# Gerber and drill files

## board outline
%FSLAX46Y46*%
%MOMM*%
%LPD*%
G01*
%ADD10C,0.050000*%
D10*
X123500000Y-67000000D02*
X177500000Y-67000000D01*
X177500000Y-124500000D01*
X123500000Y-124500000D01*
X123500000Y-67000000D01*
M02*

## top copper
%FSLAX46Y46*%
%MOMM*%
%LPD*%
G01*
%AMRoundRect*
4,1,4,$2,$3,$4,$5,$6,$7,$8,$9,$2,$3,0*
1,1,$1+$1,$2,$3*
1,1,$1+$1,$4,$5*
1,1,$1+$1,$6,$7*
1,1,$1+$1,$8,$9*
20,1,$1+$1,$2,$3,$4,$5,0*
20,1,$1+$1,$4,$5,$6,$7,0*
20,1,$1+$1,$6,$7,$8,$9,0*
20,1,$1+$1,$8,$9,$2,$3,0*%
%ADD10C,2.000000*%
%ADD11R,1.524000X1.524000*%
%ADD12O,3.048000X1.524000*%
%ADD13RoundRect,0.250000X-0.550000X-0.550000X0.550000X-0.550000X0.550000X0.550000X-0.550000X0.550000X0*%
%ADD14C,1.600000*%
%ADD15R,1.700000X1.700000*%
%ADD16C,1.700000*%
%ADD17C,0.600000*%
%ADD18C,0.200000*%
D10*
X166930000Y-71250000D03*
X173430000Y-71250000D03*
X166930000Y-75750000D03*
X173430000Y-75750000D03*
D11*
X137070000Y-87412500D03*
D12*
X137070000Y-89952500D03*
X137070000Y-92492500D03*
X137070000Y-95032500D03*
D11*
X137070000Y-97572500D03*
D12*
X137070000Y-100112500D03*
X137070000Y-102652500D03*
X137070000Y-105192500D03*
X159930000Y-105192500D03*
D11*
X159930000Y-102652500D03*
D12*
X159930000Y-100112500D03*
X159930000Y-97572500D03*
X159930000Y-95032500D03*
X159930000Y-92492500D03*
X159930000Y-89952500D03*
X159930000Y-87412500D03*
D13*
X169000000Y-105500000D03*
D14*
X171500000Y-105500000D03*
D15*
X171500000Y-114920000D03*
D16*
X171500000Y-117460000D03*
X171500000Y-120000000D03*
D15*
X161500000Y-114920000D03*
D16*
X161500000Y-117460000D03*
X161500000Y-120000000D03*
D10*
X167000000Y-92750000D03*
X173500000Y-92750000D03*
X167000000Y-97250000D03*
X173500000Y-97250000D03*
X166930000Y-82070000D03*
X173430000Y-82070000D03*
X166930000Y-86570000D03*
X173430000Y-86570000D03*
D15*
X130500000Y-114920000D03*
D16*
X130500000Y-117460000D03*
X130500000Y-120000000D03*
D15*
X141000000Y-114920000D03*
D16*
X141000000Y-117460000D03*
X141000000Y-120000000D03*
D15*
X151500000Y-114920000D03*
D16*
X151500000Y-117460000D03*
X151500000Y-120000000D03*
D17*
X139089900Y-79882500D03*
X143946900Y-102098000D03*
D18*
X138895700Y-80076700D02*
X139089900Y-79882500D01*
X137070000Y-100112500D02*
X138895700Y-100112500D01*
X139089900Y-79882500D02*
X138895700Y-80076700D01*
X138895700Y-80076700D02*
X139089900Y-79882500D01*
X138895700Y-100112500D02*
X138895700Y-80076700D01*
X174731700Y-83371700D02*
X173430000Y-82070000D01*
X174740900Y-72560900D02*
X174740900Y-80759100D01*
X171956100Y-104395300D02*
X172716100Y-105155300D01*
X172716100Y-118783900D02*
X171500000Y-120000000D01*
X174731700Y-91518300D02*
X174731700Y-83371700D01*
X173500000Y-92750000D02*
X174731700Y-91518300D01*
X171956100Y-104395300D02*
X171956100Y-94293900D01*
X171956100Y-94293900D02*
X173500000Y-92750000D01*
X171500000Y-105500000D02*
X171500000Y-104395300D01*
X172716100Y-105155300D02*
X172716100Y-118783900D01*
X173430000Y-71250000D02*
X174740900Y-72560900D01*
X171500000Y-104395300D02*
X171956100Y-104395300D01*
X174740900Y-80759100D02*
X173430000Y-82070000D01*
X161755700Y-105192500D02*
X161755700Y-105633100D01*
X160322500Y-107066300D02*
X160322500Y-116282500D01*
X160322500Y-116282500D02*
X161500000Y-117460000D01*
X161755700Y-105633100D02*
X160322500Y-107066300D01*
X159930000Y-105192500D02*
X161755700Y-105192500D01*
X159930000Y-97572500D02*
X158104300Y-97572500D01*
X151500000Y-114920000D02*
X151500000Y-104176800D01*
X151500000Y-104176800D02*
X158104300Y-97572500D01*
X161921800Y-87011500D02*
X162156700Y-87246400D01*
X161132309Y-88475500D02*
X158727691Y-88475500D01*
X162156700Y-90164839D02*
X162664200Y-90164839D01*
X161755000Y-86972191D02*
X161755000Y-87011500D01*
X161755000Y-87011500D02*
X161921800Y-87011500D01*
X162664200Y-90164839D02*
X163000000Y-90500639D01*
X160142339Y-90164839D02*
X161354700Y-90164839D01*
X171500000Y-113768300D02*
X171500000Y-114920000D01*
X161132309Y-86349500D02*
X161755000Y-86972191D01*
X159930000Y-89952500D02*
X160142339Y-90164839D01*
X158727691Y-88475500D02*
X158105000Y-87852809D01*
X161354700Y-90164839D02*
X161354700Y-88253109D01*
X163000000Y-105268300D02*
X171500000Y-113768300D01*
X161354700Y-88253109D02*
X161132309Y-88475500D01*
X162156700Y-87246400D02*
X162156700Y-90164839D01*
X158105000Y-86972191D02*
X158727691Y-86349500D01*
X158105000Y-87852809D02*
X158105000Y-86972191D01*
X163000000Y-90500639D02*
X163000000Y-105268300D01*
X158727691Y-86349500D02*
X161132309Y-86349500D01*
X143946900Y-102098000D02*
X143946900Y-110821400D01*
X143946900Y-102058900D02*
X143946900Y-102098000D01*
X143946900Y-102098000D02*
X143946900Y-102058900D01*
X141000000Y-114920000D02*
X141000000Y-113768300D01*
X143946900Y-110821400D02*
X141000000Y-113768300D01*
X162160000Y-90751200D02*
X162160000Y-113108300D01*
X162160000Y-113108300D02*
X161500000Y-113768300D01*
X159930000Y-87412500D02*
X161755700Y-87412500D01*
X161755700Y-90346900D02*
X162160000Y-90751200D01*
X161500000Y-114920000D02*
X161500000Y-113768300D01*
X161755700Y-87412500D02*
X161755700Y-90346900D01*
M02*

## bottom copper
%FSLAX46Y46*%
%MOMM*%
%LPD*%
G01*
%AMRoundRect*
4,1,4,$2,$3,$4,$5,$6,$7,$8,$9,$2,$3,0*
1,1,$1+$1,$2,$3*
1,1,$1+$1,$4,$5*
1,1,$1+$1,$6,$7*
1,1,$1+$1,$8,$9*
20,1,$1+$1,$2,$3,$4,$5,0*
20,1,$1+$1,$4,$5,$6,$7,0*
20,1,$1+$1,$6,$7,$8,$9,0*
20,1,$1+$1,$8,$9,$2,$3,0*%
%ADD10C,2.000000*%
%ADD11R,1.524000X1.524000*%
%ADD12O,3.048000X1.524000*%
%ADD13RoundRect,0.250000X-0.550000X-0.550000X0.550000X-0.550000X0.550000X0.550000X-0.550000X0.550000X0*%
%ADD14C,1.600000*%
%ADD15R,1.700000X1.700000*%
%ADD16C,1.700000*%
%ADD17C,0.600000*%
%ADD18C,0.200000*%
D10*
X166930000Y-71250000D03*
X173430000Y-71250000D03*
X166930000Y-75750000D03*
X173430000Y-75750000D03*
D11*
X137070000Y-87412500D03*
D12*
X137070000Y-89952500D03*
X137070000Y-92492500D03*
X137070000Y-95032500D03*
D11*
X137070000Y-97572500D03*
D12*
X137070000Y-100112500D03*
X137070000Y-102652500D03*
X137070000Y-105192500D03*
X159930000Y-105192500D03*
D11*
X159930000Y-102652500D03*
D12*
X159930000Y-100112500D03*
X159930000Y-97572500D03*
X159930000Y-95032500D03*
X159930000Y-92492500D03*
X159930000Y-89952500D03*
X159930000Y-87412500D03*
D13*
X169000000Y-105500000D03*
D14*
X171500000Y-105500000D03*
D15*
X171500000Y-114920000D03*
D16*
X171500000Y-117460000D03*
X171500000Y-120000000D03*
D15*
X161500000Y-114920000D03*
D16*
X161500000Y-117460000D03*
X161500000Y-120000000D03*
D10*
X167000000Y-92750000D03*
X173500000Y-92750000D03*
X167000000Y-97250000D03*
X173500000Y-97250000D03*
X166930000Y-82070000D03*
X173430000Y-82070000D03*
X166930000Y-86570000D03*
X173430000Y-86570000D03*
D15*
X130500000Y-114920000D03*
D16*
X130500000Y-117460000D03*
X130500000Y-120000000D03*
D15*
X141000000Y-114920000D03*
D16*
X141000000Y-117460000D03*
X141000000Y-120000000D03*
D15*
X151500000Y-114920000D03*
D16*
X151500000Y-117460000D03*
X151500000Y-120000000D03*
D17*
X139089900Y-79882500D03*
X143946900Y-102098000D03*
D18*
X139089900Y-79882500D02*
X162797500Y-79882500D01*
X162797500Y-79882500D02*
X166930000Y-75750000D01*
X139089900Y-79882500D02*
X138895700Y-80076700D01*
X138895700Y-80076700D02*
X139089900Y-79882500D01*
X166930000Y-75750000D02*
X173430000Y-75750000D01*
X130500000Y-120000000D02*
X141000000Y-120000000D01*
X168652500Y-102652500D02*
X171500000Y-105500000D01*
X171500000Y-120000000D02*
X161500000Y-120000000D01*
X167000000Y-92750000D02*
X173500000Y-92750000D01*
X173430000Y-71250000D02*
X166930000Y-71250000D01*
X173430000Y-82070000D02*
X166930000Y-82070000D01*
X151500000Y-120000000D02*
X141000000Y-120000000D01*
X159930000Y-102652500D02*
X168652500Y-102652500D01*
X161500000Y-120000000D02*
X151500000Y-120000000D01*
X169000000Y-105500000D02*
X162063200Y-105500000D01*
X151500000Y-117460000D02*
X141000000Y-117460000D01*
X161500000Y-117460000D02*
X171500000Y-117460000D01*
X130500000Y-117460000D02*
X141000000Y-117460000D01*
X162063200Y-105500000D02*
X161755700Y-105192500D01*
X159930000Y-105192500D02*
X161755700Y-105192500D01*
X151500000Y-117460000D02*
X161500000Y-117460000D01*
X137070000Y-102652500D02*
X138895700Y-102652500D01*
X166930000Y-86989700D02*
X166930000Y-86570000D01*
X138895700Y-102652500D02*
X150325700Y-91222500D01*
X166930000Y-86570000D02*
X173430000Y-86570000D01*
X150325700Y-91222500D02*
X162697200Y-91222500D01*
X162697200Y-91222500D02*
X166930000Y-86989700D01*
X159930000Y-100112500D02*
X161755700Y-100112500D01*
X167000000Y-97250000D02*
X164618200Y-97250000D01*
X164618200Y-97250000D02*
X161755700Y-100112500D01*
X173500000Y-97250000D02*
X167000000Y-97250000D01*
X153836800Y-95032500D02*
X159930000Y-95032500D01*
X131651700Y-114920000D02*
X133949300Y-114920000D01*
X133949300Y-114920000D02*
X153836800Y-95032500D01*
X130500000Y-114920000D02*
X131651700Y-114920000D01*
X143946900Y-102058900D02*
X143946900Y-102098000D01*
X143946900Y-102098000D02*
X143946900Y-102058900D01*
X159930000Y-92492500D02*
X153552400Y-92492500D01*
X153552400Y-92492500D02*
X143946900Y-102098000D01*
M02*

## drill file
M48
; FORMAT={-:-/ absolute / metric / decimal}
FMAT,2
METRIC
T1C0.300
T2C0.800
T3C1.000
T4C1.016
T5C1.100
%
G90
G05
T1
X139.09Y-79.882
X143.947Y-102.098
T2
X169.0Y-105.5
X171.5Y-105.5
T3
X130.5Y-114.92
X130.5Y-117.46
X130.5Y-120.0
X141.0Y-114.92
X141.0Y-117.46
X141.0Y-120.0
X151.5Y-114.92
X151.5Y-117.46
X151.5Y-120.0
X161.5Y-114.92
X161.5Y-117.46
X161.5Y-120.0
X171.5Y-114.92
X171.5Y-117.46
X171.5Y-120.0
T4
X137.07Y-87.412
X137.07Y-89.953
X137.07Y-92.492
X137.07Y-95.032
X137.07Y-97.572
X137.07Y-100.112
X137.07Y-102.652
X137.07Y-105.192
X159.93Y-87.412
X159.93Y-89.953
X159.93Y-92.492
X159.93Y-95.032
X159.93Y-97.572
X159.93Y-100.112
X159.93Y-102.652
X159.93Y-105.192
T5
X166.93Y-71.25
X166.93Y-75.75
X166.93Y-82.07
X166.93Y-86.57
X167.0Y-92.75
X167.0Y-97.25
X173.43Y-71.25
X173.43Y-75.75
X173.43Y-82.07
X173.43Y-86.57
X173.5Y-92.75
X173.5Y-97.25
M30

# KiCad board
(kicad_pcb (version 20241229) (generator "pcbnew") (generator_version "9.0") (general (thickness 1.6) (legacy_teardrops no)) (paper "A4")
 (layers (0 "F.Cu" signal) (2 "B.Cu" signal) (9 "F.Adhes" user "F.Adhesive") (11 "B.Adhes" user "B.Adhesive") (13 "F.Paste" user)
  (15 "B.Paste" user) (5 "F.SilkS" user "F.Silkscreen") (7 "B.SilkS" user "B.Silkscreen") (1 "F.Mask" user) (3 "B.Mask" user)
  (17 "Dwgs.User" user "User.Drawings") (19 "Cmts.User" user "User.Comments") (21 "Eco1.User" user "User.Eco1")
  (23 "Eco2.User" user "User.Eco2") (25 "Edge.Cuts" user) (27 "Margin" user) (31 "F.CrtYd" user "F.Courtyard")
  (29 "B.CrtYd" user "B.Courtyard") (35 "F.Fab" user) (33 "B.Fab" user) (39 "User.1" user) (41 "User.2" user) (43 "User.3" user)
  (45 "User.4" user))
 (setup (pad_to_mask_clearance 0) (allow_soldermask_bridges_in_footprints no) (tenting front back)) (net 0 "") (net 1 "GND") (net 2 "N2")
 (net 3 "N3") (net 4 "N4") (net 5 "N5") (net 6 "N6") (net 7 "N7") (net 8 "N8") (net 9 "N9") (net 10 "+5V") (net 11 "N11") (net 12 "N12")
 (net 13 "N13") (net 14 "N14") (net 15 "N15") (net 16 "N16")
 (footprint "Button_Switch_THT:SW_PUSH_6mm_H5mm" (layer "F.Cu") (at 166.93 71.25)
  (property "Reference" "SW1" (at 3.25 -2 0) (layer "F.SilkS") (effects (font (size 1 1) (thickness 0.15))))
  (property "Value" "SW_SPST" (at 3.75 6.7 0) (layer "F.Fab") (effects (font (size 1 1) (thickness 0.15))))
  (pad "1" thru_hole circle (at 0 0 90) (size 2 2) (drill 1.1) (layers "*.Cu" "*.Mask") (remove_unused_layers no) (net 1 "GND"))
  (pad "1" thru_hole circle (at 6.5 0 90) (size 2 2) (drill 1.1) (layers "*.Cu" "*.Mask") (remove_unused_layers no) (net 1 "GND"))
  (pad "2" thru_hole circle (at 0 4.5 90) (size 2 2) (drill 1.1) (layers "*.Cu" "*.Mask") (remove_unused_layers no) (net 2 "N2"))
  (pad "2" thru_hole circle (at 6.5 4.5 90) (size 2 2) (drill 1.1) (layers "*.Cu" "*.Mask") (remove_unused_layers no) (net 2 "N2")))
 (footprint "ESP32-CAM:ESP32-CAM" (layer "F.Cu") (at 148.5 95.0325)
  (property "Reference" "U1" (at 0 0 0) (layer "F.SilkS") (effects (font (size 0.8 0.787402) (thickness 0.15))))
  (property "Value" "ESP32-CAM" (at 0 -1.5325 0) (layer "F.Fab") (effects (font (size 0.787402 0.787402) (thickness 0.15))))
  (pad "P$1" thru_hole rect (at -11.43 -7.62) (size 1.524 1.524) (drill 1.016) (layers "*.Cu" "*.Mask") (remove_unused_layers no)
   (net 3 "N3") (solder_mask_margin 0.102))
  (pad "P$2" thru_hole oval (at -11.43 -5.08) (size 3.048 1.524) (drill 1.016) (layers "*.Cu" "*.Mask") (remove_unused_layers no)
   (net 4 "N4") (solder_mask_margin 0.102))
  (pad "P$3" thru_hole oval (at -11.43 -2.54) (size 3.048 1.524) (drill 1.016) (layers "*.Cu" "*.Mask") (remove_unused_layers no)
   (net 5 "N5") (solder_mask_margin 0.102))
  (pad "P$4" thru_hole oval (at -11.43 0) (size 3.048 1.524) (drill 1.016) (layers "*.Cu" "*.Mask") (remove_unused_layers no) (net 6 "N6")
   (solder_mask_margin 0.102))
  (pad "P$5" thru_hole rect (at -11.43 2.54) (size 1.524 1.524) (drill 1.016) (layers "*.Cu" "*.Mask") (remove_unused_layers no)
   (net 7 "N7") (solder_mask_margin 0.102))
  (pad "P$6" thru_hole oval (at -11.43 5.08) (size 3.048 1.524) (drill 1.016) (layers "*.Cu" "*.Mask") (remove_unused_layers no)
   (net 2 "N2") (solder_mask_margin 0.102))
  (pad "P$7" thru_hole oval (at -11.43 7.62) (size 3.048 1.524) (drill 1.016) (layers "*.Cu" "*.Mask") (remove_unused_layers no)
   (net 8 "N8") (solder_mask_margin 0.102))
  (pad "P$8" thru_hole oval (at -11.43 10.16) (size 3.048 1.524) (drill 1.016) (layers "*.Cu" "*.Mask") (remove_unused_layers no)
   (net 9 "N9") (solder_mask_margin 0.102))
  (pad "P$9" thru_hole oval (at 11.43 10.16) (size 3.048 1.524) (drill 1.016) (layers "*.Cu" "*.Mask") (remove_unused_layers no)
   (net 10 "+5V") (solder_mask_margin 0.102))
  (pad "P$10" thru_hole rect (at 11.43 7.62) (size 1.524 1.524) (drill 1.016) (layers "*.Cu" "*.Mask") (remove_unused_layers no)
   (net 1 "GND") (solder_mask_margin 0.102))
  (pad "P$11" thru_hole oval (at 11.43 5.08) (size 3.048 1.524) (drill 1.016) (layers "*.Cu" "*.Mask") (remove_unused_layers no)
   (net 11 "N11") (solder_mask_margin 0.102))
  (pad "P$12" thru_hole oval (at 11.43 2.54) (size 3.048 1.524) (drill 1.016) (layers "*.Cu" "*.Mask") (remove_unused_layers no)
   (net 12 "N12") (solder_mask_margin 0.102))
  (pad "P$13" thru_hole oval (at 11.43 0) (size 3.048 1.524) (drill 1.016) (layers "*.Cu" "*.Mask") (remove_unused_layers no) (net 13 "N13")
   (solder_mask_margin 0.102))
  (pad "P$14" thru_hole oval (at 11.43 -2.54) (size 3.048 1.524) (drill 1.016) (layers "*.Cu" "*.Mask") (remove_unused_layers no)
   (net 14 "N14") (solder_mask_margin 0.102))
  (pad "P$15" thru_hole oval (at 11.43 -5.08) (size 3.048 1.524) (drill 1.016) (layers "*.Cu" "*.Mask") (remove_unused_layers no)
   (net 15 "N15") (solder_mask_margin 0.102))
  (pad "P$16" thru_hole oval (at 11.43 -7.62) (size 3.048 1.524) (drill 1.016) (layers "*.Cu" "*.Mask") (remove_unused_layers no)
   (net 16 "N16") (solder_mask_margin 0.102)))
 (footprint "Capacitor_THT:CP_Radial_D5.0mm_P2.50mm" (layer "F.Cu") (at 169 105.5)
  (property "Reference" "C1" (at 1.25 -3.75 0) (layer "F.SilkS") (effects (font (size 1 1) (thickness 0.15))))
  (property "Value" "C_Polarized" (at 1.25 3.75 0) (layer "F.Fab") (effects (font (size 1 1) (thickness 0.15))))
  (pad "1" thru_hole roundrect (at 0 0) (size 1.6 1.6) (drill 0.8) (layers "*.Cu" "*.Mask") (remove_unused_layers no)
   (roundrect_rratio 0.15625) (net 10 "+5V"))
  (pad "2" thru_hole circle (at 2.5 0) (size 1.6 1.6) (drill 0.8) (layers "*.Cu" "*.Mask") (remove_unused_layers no) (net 1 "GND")))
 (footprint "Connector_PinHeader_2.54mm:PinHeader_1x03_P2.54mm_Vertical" (layer "F.Cu") (at 171.5 114.92)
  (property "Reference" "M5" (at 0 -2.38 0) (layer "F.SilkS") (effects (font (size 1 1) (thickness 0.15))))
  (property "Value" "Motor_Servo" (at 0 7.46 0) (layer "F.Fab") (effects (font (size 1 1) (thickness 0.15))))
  (pad "1" thru_hole rect (at 0 0) (size 1.7 1.7) (drill 1) (layers "*.Cu" "*.Mask") (remove_unused_layers no) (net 15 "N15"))
  (pad "2" thru_hole circle (at 0 2.54) (size 1.7 1.7) (drill 1) (layers "*.Cu" "*.Mask") (remove_unused_layers no) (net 10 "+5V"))
  (pad "3" thru_hole circle (at 0 5.08) (size 1.7 1.7) (drill 1) (layers "*.Cu" "*.Mask") (remove_unused_layers no) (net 1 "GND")))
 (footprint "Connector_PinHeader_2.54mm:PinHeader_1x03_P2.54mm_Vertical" (layer "F.Cu") (at 161.5 114.92)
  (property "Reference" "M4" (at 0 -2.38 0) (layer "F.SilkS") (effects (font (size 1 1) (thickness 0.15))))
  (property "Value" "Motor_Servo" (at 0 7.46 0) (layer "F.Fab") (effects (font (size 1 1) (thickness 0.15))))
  (pad "1" thru_hole rect (at 0 0) (size 1.7 1.7) (drill 1) (layers "*.Cu" "*.Mask") (remove_unused_layers no) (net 16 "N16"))
  (pad "2" thru_hole circle (at 0 2.54) (size 1.7 1.7) (drill 1) (layers "*.Cu" "*.Mask") (remove_unused_layers no) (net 10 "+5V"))
  (pad "3" thru_hole circle (at 0 5.08) (size 1.7 1.7) (drill 1) (layers "*.Cu" "*.Mask") (remove_unused_layers no) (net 1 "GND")))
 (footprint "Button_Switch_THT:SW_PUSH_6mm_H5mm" (layer "F.Cu") (at 167 92.75)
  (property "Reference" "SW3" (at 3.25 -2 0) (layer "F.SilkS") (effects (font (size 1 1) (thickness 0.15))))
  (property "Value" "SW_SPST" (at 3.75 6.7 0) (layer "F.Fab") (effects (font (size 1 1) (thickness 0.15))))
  (pad "1" thru_hole circle (at 0 0 90) (size 2 2) (drill 1.1) (layers "*.Cu" "*.Mask") (remove_unused_layers no) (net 1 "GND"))
  (pad "1" thru_hole circle (at 6.5 0 90) (size 2 2) (drill 1.1) (layers "*.Cu" "*.Mask") (remove_unused_layers no) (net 1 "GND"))
  (pad "2" thru_hole circle (at 0 4.5 90) (size 2 2) (drill 1.1) (layers "*.Cu" "*.Mask") (remove_unused_layers no) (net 11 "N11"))
  (pad "2" thru_hole circle (at 6.5 4.5 90) (size 2 2) (drill 1.1) (layers "*.Cu" "*.Mask") (remove_unused_layers no) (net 11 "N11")))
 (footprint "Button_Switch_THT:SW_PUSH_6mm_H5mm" (layer "F.Cu") (at 166.93 82.07)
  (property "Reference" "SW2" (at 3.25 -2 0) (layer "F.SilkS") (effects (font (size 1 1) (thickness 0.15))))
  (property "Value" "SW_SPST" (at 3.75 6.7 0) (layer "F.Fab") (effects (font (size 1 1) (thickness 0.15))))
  (pad "1" thru_hole circle (at 0 0 90) (size 2 2) (drill 1.1) (layers "*.Cu" "*.Mask") (remove_unused_layers no) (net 1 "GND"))
  (pad "1" thru_hole circle (at 6.5 0 90) (size 2 2) (drill 1.1) (layers "*.Cu" "*.Mask") (remove_unused_layers no) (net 1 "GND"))
  (pad "2" thru_hole circle (at 0 4.5 90) (size 2 2) (drill 1.1) (layers "*.Cu" "*.Mask") (remove_unused_layers no) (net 8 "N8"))
  (pad "2" thru_hole circle (at 6.5 4.5 90) (size 2 2) (drill 1.1) (layers "*.Cu" "*.Mask") (remove_unused_layers no) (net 8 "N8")))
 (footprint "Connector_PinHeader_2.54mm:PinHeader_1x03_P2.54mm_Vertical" (layer "F.Cu") (at 130.5 114.92)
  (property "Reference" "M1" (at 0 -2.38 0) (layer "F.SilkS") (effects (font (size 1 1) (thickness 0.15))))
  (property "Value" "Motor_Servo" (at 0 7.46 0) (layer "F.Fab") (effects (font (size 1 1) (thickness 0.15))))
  (pad "1" thru_hole rect (at 0 0) (size 1.7 1.7) (drill 1) (layers "*.Cu" "*.Mask") (remove_unused_layers no) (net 13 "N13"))
  (pad "2" thru_hole circle (at 0 2.54) (size 1.7 1.7) (drill 1) (layers "*.Cu" "*.Mask") (remove_unused_layers no) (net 10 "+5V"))
  (pad "3" thru_hole circle (at 0 5.08) (size 1.7 1.7) (drill 1) (layers "*.Cu" "*.Mask") (remove_unused_layers no) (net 1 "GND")))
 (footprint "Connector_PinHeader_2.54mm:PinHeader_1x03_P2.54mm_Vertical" (layer "F.Cu") (at 141 114.92)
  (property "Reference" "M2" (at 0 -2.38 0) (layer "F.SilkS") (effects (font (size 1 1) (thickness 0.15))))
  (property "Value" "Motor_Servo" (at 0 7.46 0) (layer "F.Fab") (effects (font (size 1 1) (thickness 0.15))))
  (pad "1" thru_hole rect (at 0 0) (size 1.7 1.7) (drill 1) (layers "*.Cu" "*.Mask") (remove_unused_layers no) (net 14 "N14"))
  (pad "2" thru_hole circle (at 0 2.54) (size 1.7 1.7) (drill 1) (layers "*.Cu" "*.Mask") (remove_unused_layers no) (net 10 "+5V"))
  (pad "3" thru_hole circle (at 0 5.08) (size 1.7 1.7) (drill 1) (layers "*.Cu" "*.Mask") (remove_unused_layers no) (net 1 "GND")))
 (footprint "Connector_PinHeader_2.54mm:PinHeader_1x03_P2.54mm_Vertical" (layer "F.Cu") (at 151.5 114.92)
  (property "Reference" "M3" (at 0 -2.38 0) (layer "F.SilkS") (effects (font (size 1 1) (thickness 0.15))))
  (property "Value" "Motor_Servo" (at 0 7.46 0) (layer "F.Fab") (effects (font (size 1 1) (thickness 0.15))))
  (pad "1" thru_hole rect (at 0 0) (size 1.7 1.7) (drill 1) (layers "*.Cu" "*.Mask") (remove_unused_layers no) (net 12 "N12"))
  (pad "2" thru_hole circle (at 0 2.54) (size 1.7 1.7) (drill 1) (layers "*.Cu" "*.Mask") (remove_unused_layers no) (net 10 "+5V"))
  (pad "3" thru_hole circle (at 0 5.08) (size 1.7 1.7) (drill 1) (layers "*.Cu" "*.Mask") (remove_unused_layers no) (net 1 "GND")))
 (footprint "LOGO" (layer "B.Cu") (at 129.5 77.5 -90)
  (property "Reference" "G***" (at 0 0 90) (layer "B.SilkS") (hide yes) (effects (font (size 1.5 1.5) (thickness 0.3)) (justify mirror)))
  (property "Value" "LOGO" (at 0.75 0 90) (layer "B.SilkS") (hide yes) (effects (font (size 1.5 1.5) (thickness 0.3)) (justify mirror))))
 (gr_rect (start 123.5 67) (end 177.5 124.5) (stroke (width 0.05) (type default)) (fill no) (layer "Edge.Cuts"))
 (segment (start 138.8957 80.0767) (end 139.0899 79.8825) (width 0.2) (layer "F.Cu") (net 2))
 (segment (start 137.07 100.1125) (end 138.8957 100.1125) (width 0.2) (layer "F.Cu") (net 2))
 (segment (start 139.0899 79.8825) (end 138.8957 80.0767) (width 0.2) (layer "F.Cu") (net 2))
 (segment (start 138.8957 80.0767) (end 139.0899 79.8825) (width 0.2) (layer "F.Cu") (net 2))
 (segment (start 138.8957 100.1125) (end 138.8957 80.0767) (width 0.2) (layer "F.Cu") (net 2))
 (via (at 139.0899 79.8825) (size 0.6) (drill 0.3) (layers "F.Cu" "B.Cu") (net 2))
 (segment (start 139.0899 79.8825) (end 162.7975 79.8825) (width 0.2) (layer "B.Cu") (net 2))
 (segment (start 162.7975 79.8825) (end 166.93 75.75) (width 0.2) (layer "B.Cu") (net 2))
 (segment (start 139.0899 79.8825) (end 138.8957 80.0767) (width 0.2) (layer "B.Cu") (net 2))
 (segment (start 138.8957 80.0767) (end 139.0899 79.8825) (width 0.2) (layer "B.Cu") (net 2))
 (segment (start 166.93 75.75) (end 173.43 75.75) (width 0.2) (layer "B.Cu") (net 2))
 (segment (start 174.7317 83.3717) (end 173.43 82.07) (width 0.2) (layer "F.Cu") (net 1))
 (segment (start 174.7409 72.5609) (end 174.7409 80.7591) (width 0.2) (layer "F.Cu") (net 1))
 (segment (start 171.9561 104.3953) (end 172.7161 105.1553) (width 0.2) (layer "F.Cu") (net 1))
 (segment (start 172.7161 118.7839) (end 171.5 120) (width 0.2) (layer "F.Cu") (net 1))
 (segment (start 174.7317 91.5183) (end 174.7317 83.3717) (width 0.2) (layer "F.Cu") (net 1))
 (segment (start 173.5 92.75) (end 174.7317 91.5183) (width 0.2) (layer "F.Cu") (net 1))
 (segment (start 171.9561 104.3953) (end 171.9561 94.2939) (width 0.2) (layer "F.Cu") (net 1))
 (segment (start 171.9561 94.2939) (end 173.5 92.75) (width 0.2) (layer "F.Cu") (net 1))
 (segment (start 171.5 105.5) (end 171.5 104.3953) (width 0.2) (layer "F.Cu") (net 1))
 (segment (start 172.7161 105.1553) (end 172.7161 118.7839) (width 0.2) (layer "F.Cu") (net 1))
 (segment (start 173.43 71.25) (end 174.7409 72.5609) (width 0.2) (layer "F.Cu") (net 1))
 (segment (start 171.5 104.3953) (end 171.9561 104.3953) (width 0.2) (layer "F.Cu") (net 1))
 (segment (start 174.7409 80.7591) (end 173.43 82.07) (width 0.2) (layer "F.Cu") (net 1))
 (segment (start 130.5 120) (end 141 120) (width 0.2) (layer "B.Cu") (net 1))
 (segment (start 168.6525 102.6525) (end 171.5 105.5) (width 0.2) (layer "B.Cu") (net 1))
 (segment (start 171.5 120) (end 161.5 120) (width 0.2) (layer "B.Cu") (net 1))
 (segment (start 167 92.75) (end 173.5 92.75) (width 0.2) (layer "B.Cu") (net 1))
 (segment (start 173.43 71.25) (end 166.93 71.25) (width 0.2) (layer "B.Cu") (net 1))
 (segment (start 173.43 82.07) (end 166.93 82.07) (width 0.2) (layer "B.Cu") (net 1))
 (segment (start 151.5 120) (end 141 120) (width 0.2) (layer "B.Cu") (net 1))
 (segment (start 159.93 102.6525) (end 168.6525 102.6525) (width 0.2) (layer "B.Cu") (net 1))
 (segment (start 161.5 120) (end 151.5 120) (width 0.2) (layer "B.Cu") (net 1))
 (segment (start 161.7557 105.1925) (end 161.7557 105.6331) (width 0.2) (layer "F.Cu") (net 10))
 (segment (start 160.3225 107.0663) (end 160.3225 116.2825) (width 0.2) (layer "F.Cu") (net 10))
 (segment (start 160.3225 116.2825) (end 161.5 117.46) (width 0.2) (layer "F.Cu") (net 10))
 (segment (start 161.7557 105.6331) (end 160.3225 107.0663) (width 0.2) (layer "F.Cu") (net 10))
 (segment (start 159.93 105.1925) (end 161.7557 105.1925) (width 0.2) (layer "F.Cu") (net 10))
 (segment (start 169 105.5) (end 162.0632 105.5) (width 0.2) (layer "B.Cu") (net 10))
 (segment (start 151.5 117.46) (end 141 117.46) (width 0.2) (layer "B.Cu") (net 10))
 (segment (start 161.5 117.46) (end 171.5 117.46) (width 0.2) (layer "B.Cu") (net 10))
 (segment (start 130.5 117.46) (end 141 117.46) (width 0.2) (layer "B.Cu") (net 10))
 (segment (start 162.0632 105.5) (end 161.7557 105.1925) (width 0.2) (layer "B.Cu") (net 10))
 (segment (start 159.93 105.1925) (end 161.7557 105.1925) (width 0.2) (layer "B.Cu") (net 10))
 (segment (start 151.5 117.46) (end 161.5 117.46) (width 0.2) (layer "B.Cu") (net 10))
 (segment (start 137.07 102.6525) (end 138.8957 102.6525) (width 0.2) (layer "B.Cu") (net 8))
 (segment (start 166.93 86.9897) (end 166.93 86.57) (width 0.2) (layer "B.Cu") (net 8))
 (segment (start 138.8957 102.6525) (end 150.3257 91.2225) (width 0.2) (layer "B.Cu") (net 8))
 (segment (start 166.93 86.57) (end 173.43 86.57) (width 0.2) (layer "B.Cu") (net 8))
 (segment (start 150.3257 91.2225) (end 162.6972 91.2225) (width 0.2) (layer "B.Cu") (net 8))
 (segment (start 162.6972 91.2225) (end 166.93 86.9897) (width 0.2) (layer "B.Cu") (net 8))
 (segment (start 159.93 100.1125) (end 161.7557 100.1125) (width 0.2) (layer "B.Cu") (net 11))
 (segment (start 167 97.25) (end 164.6182 97.25) (width 0.2) (layer "B.Cu") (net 11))
 (segment (start 164.6182 97.25) (end 161.7557 100.1125) (width 0.2) (layer "B.Cu") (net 11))
 (segment (start 173.5 97.25) (end 167 97.25) (width 0.2) (layer "B.Cu") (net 11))
 (segment (start 159.93 97.5725) (end 158.1043 97.5725) (width 0.2) (layer "F.Cu") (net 12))
 (segment (start 151.5 114.92) (end 151.5 104.1768) (width 0.2) (layer "F.Cu") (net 12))
 (segment (start 151.5 104.1768) (end 158.1043 97.5725) (width 0.2) (layer "F.Cu") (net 12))
 (segment (start 153.8368 95.0325) (end 159.93 95.0325) (width 0.2) (layer "B.Cu") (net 13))
 (segment (start 131.6517 114.92) (end 133.9493 114.92) (width 0.2) (layer "B.Cu") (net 13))
 (segment (start 133.9493 114.92) (end 153.8368 95.0325) (width 0.2) (layer "B.Cu") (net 13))
 (segment (start 130.5 114.92) (end 131.6517 114.92) (width 0.2) (layer "B.Cu") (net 13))
 (segment (start 161.9218 87.0115) (end 162.1567 87.2464) (width 0.2) (layer "F.Cu") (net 15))
 (segment (start 161.132309 88.4755) (end 158.727691 88.4755) (width 0.2) (layer "F.Cu") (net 15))
 (segment (start 162.1567 90.164839) (end 162.6642 90.164839) (width 0.2) (layer "F.Cu") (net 15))
 (segment (start 161.755 86.972191) (end 161.755 87.0115) (width 0.2) (layer "F.Cu") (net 15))
 (segment (start 161.755 87.0115) (end 161.9218 87.0115) (width 0.2) (layer "F.Cu") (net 15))
 (segment (start 162.6642 90.164839) (end 163 90.500639) (width 0.2) (layer "F.Cu") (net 15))
 (segment (start 160.142339 90.164839) (end 161.3547 90.164839) (width 0.2) (layer "F.Cu") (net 15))
 (segment (start 171.5 113.7683) (end 171.5 114.92) (width 0.2) (layer "F.Cu") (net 15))
 (segment (start 161.132309 86.3495) (end 161.755 86.972191) (width 0.2) (layer "F.Cu") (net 15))
 (segment (start 159.93 89.9525) (end 160.142339 90.164839) (width 0.2) (layer "F.Cu") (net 15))
 (segment (start 158.727691 88.4755) (end 158.105 87.852809) (width 0.2) (layer "F.Cu") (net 15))
 (segment (start 161.3547 90.164839) (end 161.3547 88.253109) (width 0.2) (layer "F.Cu") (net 15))
 (segment (start 163 105.2683) (end 171.5 113.7683) (width 0.2) (layer "F.Cu") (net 15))
 (segment (start 161.3547 88.253109) (end 161.132309 88.4755) (width 0.2) (layer "F.Cu") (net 15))
 (segment (start 162.1567 87.2464) (end 162.1567 90.164839) (width 0.2) (layer "F.Cu") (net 15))
 (segment (start 158.105 86.972191) (end 158.727691 86.3495) (width 0.2) (layer "F.Cu") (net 15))
 (segment (start 158.105 87.852809) (end 158.105 86.972191) (width 0.2) (layer "F.Cu") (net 15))
 (segment (start 163 90.500639) (end 163 105.2683) (width 0.2) (layer "F.Cu") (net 15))
 (segment (start 158.727691 86.3495) (end 161.132309 86.3495) (width 0.2) (layer "F.Cu") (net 15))
 (segment (start 143.9469 102.098) (end 143.9469 110.8214) (width 0.2) (layer "F.Cu") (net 14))
 (segment (start 143.9469 102.0589) (end 143.9469 102.098) (width 0.2) (layer "F.Cu") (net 14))
 (segment (start 143.9469 102.098) (end 143.9469 102.0589) (width 0.2) (layer "F.Cu") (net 14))
 (segment (start 141 114.92) (end 141 113.7683) (width 0.2) (layer "F.Cu") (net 14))
 (segment (start 143.9469 110.8214) (end 141 113.7683) (width 0.2) (layer "F.Cu") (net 14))
 (via (at 143.9469 102.098) (size 0.6) (drill 0.3) (layers "F.Cu" "B.Cu") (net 14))
 (segment (start 143.9469 102.0589) (end 143.9469 102.098) (width 0.2) (layer "B.Cu") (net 14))
 (segment (start 143.9469 102.098) (end 143.9469 102.0589) (width 0.2) (layer "B.Cu") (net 14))
 (segment (start 159.93 92.4925) (end 153.5524 92.4925) (width 0.2) (layer "B.Cu") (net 14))
 (segment (start 153.5524 92.4925) (end 143.9469 102.098) (width 0.2) (layer "B.Cu") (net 14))
 (segment (start 162.16 90.7512) (end 162.16 113.1083) (width 0.2) (layer "F.Cu") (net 16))
 (segment (start 162.16 113.1083) (end 161.5 113.7683) (width 0.2) (layer "F.Cu") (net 16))
 (segment (start 159.93 87.4125) (end 161.7557 87.4125) (width 0.2) (layer "F.Cu") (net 16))
 (segment (start 161.7557 90.3469) (end 162.16 90.7512) (width 0.2) (layer "F.Cu") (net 16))
 (segment (start 161.5 114.92) (end 161.5 113.7683) (width 0.2) (layer "F.Cu") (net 16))
 (segment (start 161.7557 87.4125) (end 161.7557 90.3469) (width 0.2) (layer "F.Cu") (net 16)))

